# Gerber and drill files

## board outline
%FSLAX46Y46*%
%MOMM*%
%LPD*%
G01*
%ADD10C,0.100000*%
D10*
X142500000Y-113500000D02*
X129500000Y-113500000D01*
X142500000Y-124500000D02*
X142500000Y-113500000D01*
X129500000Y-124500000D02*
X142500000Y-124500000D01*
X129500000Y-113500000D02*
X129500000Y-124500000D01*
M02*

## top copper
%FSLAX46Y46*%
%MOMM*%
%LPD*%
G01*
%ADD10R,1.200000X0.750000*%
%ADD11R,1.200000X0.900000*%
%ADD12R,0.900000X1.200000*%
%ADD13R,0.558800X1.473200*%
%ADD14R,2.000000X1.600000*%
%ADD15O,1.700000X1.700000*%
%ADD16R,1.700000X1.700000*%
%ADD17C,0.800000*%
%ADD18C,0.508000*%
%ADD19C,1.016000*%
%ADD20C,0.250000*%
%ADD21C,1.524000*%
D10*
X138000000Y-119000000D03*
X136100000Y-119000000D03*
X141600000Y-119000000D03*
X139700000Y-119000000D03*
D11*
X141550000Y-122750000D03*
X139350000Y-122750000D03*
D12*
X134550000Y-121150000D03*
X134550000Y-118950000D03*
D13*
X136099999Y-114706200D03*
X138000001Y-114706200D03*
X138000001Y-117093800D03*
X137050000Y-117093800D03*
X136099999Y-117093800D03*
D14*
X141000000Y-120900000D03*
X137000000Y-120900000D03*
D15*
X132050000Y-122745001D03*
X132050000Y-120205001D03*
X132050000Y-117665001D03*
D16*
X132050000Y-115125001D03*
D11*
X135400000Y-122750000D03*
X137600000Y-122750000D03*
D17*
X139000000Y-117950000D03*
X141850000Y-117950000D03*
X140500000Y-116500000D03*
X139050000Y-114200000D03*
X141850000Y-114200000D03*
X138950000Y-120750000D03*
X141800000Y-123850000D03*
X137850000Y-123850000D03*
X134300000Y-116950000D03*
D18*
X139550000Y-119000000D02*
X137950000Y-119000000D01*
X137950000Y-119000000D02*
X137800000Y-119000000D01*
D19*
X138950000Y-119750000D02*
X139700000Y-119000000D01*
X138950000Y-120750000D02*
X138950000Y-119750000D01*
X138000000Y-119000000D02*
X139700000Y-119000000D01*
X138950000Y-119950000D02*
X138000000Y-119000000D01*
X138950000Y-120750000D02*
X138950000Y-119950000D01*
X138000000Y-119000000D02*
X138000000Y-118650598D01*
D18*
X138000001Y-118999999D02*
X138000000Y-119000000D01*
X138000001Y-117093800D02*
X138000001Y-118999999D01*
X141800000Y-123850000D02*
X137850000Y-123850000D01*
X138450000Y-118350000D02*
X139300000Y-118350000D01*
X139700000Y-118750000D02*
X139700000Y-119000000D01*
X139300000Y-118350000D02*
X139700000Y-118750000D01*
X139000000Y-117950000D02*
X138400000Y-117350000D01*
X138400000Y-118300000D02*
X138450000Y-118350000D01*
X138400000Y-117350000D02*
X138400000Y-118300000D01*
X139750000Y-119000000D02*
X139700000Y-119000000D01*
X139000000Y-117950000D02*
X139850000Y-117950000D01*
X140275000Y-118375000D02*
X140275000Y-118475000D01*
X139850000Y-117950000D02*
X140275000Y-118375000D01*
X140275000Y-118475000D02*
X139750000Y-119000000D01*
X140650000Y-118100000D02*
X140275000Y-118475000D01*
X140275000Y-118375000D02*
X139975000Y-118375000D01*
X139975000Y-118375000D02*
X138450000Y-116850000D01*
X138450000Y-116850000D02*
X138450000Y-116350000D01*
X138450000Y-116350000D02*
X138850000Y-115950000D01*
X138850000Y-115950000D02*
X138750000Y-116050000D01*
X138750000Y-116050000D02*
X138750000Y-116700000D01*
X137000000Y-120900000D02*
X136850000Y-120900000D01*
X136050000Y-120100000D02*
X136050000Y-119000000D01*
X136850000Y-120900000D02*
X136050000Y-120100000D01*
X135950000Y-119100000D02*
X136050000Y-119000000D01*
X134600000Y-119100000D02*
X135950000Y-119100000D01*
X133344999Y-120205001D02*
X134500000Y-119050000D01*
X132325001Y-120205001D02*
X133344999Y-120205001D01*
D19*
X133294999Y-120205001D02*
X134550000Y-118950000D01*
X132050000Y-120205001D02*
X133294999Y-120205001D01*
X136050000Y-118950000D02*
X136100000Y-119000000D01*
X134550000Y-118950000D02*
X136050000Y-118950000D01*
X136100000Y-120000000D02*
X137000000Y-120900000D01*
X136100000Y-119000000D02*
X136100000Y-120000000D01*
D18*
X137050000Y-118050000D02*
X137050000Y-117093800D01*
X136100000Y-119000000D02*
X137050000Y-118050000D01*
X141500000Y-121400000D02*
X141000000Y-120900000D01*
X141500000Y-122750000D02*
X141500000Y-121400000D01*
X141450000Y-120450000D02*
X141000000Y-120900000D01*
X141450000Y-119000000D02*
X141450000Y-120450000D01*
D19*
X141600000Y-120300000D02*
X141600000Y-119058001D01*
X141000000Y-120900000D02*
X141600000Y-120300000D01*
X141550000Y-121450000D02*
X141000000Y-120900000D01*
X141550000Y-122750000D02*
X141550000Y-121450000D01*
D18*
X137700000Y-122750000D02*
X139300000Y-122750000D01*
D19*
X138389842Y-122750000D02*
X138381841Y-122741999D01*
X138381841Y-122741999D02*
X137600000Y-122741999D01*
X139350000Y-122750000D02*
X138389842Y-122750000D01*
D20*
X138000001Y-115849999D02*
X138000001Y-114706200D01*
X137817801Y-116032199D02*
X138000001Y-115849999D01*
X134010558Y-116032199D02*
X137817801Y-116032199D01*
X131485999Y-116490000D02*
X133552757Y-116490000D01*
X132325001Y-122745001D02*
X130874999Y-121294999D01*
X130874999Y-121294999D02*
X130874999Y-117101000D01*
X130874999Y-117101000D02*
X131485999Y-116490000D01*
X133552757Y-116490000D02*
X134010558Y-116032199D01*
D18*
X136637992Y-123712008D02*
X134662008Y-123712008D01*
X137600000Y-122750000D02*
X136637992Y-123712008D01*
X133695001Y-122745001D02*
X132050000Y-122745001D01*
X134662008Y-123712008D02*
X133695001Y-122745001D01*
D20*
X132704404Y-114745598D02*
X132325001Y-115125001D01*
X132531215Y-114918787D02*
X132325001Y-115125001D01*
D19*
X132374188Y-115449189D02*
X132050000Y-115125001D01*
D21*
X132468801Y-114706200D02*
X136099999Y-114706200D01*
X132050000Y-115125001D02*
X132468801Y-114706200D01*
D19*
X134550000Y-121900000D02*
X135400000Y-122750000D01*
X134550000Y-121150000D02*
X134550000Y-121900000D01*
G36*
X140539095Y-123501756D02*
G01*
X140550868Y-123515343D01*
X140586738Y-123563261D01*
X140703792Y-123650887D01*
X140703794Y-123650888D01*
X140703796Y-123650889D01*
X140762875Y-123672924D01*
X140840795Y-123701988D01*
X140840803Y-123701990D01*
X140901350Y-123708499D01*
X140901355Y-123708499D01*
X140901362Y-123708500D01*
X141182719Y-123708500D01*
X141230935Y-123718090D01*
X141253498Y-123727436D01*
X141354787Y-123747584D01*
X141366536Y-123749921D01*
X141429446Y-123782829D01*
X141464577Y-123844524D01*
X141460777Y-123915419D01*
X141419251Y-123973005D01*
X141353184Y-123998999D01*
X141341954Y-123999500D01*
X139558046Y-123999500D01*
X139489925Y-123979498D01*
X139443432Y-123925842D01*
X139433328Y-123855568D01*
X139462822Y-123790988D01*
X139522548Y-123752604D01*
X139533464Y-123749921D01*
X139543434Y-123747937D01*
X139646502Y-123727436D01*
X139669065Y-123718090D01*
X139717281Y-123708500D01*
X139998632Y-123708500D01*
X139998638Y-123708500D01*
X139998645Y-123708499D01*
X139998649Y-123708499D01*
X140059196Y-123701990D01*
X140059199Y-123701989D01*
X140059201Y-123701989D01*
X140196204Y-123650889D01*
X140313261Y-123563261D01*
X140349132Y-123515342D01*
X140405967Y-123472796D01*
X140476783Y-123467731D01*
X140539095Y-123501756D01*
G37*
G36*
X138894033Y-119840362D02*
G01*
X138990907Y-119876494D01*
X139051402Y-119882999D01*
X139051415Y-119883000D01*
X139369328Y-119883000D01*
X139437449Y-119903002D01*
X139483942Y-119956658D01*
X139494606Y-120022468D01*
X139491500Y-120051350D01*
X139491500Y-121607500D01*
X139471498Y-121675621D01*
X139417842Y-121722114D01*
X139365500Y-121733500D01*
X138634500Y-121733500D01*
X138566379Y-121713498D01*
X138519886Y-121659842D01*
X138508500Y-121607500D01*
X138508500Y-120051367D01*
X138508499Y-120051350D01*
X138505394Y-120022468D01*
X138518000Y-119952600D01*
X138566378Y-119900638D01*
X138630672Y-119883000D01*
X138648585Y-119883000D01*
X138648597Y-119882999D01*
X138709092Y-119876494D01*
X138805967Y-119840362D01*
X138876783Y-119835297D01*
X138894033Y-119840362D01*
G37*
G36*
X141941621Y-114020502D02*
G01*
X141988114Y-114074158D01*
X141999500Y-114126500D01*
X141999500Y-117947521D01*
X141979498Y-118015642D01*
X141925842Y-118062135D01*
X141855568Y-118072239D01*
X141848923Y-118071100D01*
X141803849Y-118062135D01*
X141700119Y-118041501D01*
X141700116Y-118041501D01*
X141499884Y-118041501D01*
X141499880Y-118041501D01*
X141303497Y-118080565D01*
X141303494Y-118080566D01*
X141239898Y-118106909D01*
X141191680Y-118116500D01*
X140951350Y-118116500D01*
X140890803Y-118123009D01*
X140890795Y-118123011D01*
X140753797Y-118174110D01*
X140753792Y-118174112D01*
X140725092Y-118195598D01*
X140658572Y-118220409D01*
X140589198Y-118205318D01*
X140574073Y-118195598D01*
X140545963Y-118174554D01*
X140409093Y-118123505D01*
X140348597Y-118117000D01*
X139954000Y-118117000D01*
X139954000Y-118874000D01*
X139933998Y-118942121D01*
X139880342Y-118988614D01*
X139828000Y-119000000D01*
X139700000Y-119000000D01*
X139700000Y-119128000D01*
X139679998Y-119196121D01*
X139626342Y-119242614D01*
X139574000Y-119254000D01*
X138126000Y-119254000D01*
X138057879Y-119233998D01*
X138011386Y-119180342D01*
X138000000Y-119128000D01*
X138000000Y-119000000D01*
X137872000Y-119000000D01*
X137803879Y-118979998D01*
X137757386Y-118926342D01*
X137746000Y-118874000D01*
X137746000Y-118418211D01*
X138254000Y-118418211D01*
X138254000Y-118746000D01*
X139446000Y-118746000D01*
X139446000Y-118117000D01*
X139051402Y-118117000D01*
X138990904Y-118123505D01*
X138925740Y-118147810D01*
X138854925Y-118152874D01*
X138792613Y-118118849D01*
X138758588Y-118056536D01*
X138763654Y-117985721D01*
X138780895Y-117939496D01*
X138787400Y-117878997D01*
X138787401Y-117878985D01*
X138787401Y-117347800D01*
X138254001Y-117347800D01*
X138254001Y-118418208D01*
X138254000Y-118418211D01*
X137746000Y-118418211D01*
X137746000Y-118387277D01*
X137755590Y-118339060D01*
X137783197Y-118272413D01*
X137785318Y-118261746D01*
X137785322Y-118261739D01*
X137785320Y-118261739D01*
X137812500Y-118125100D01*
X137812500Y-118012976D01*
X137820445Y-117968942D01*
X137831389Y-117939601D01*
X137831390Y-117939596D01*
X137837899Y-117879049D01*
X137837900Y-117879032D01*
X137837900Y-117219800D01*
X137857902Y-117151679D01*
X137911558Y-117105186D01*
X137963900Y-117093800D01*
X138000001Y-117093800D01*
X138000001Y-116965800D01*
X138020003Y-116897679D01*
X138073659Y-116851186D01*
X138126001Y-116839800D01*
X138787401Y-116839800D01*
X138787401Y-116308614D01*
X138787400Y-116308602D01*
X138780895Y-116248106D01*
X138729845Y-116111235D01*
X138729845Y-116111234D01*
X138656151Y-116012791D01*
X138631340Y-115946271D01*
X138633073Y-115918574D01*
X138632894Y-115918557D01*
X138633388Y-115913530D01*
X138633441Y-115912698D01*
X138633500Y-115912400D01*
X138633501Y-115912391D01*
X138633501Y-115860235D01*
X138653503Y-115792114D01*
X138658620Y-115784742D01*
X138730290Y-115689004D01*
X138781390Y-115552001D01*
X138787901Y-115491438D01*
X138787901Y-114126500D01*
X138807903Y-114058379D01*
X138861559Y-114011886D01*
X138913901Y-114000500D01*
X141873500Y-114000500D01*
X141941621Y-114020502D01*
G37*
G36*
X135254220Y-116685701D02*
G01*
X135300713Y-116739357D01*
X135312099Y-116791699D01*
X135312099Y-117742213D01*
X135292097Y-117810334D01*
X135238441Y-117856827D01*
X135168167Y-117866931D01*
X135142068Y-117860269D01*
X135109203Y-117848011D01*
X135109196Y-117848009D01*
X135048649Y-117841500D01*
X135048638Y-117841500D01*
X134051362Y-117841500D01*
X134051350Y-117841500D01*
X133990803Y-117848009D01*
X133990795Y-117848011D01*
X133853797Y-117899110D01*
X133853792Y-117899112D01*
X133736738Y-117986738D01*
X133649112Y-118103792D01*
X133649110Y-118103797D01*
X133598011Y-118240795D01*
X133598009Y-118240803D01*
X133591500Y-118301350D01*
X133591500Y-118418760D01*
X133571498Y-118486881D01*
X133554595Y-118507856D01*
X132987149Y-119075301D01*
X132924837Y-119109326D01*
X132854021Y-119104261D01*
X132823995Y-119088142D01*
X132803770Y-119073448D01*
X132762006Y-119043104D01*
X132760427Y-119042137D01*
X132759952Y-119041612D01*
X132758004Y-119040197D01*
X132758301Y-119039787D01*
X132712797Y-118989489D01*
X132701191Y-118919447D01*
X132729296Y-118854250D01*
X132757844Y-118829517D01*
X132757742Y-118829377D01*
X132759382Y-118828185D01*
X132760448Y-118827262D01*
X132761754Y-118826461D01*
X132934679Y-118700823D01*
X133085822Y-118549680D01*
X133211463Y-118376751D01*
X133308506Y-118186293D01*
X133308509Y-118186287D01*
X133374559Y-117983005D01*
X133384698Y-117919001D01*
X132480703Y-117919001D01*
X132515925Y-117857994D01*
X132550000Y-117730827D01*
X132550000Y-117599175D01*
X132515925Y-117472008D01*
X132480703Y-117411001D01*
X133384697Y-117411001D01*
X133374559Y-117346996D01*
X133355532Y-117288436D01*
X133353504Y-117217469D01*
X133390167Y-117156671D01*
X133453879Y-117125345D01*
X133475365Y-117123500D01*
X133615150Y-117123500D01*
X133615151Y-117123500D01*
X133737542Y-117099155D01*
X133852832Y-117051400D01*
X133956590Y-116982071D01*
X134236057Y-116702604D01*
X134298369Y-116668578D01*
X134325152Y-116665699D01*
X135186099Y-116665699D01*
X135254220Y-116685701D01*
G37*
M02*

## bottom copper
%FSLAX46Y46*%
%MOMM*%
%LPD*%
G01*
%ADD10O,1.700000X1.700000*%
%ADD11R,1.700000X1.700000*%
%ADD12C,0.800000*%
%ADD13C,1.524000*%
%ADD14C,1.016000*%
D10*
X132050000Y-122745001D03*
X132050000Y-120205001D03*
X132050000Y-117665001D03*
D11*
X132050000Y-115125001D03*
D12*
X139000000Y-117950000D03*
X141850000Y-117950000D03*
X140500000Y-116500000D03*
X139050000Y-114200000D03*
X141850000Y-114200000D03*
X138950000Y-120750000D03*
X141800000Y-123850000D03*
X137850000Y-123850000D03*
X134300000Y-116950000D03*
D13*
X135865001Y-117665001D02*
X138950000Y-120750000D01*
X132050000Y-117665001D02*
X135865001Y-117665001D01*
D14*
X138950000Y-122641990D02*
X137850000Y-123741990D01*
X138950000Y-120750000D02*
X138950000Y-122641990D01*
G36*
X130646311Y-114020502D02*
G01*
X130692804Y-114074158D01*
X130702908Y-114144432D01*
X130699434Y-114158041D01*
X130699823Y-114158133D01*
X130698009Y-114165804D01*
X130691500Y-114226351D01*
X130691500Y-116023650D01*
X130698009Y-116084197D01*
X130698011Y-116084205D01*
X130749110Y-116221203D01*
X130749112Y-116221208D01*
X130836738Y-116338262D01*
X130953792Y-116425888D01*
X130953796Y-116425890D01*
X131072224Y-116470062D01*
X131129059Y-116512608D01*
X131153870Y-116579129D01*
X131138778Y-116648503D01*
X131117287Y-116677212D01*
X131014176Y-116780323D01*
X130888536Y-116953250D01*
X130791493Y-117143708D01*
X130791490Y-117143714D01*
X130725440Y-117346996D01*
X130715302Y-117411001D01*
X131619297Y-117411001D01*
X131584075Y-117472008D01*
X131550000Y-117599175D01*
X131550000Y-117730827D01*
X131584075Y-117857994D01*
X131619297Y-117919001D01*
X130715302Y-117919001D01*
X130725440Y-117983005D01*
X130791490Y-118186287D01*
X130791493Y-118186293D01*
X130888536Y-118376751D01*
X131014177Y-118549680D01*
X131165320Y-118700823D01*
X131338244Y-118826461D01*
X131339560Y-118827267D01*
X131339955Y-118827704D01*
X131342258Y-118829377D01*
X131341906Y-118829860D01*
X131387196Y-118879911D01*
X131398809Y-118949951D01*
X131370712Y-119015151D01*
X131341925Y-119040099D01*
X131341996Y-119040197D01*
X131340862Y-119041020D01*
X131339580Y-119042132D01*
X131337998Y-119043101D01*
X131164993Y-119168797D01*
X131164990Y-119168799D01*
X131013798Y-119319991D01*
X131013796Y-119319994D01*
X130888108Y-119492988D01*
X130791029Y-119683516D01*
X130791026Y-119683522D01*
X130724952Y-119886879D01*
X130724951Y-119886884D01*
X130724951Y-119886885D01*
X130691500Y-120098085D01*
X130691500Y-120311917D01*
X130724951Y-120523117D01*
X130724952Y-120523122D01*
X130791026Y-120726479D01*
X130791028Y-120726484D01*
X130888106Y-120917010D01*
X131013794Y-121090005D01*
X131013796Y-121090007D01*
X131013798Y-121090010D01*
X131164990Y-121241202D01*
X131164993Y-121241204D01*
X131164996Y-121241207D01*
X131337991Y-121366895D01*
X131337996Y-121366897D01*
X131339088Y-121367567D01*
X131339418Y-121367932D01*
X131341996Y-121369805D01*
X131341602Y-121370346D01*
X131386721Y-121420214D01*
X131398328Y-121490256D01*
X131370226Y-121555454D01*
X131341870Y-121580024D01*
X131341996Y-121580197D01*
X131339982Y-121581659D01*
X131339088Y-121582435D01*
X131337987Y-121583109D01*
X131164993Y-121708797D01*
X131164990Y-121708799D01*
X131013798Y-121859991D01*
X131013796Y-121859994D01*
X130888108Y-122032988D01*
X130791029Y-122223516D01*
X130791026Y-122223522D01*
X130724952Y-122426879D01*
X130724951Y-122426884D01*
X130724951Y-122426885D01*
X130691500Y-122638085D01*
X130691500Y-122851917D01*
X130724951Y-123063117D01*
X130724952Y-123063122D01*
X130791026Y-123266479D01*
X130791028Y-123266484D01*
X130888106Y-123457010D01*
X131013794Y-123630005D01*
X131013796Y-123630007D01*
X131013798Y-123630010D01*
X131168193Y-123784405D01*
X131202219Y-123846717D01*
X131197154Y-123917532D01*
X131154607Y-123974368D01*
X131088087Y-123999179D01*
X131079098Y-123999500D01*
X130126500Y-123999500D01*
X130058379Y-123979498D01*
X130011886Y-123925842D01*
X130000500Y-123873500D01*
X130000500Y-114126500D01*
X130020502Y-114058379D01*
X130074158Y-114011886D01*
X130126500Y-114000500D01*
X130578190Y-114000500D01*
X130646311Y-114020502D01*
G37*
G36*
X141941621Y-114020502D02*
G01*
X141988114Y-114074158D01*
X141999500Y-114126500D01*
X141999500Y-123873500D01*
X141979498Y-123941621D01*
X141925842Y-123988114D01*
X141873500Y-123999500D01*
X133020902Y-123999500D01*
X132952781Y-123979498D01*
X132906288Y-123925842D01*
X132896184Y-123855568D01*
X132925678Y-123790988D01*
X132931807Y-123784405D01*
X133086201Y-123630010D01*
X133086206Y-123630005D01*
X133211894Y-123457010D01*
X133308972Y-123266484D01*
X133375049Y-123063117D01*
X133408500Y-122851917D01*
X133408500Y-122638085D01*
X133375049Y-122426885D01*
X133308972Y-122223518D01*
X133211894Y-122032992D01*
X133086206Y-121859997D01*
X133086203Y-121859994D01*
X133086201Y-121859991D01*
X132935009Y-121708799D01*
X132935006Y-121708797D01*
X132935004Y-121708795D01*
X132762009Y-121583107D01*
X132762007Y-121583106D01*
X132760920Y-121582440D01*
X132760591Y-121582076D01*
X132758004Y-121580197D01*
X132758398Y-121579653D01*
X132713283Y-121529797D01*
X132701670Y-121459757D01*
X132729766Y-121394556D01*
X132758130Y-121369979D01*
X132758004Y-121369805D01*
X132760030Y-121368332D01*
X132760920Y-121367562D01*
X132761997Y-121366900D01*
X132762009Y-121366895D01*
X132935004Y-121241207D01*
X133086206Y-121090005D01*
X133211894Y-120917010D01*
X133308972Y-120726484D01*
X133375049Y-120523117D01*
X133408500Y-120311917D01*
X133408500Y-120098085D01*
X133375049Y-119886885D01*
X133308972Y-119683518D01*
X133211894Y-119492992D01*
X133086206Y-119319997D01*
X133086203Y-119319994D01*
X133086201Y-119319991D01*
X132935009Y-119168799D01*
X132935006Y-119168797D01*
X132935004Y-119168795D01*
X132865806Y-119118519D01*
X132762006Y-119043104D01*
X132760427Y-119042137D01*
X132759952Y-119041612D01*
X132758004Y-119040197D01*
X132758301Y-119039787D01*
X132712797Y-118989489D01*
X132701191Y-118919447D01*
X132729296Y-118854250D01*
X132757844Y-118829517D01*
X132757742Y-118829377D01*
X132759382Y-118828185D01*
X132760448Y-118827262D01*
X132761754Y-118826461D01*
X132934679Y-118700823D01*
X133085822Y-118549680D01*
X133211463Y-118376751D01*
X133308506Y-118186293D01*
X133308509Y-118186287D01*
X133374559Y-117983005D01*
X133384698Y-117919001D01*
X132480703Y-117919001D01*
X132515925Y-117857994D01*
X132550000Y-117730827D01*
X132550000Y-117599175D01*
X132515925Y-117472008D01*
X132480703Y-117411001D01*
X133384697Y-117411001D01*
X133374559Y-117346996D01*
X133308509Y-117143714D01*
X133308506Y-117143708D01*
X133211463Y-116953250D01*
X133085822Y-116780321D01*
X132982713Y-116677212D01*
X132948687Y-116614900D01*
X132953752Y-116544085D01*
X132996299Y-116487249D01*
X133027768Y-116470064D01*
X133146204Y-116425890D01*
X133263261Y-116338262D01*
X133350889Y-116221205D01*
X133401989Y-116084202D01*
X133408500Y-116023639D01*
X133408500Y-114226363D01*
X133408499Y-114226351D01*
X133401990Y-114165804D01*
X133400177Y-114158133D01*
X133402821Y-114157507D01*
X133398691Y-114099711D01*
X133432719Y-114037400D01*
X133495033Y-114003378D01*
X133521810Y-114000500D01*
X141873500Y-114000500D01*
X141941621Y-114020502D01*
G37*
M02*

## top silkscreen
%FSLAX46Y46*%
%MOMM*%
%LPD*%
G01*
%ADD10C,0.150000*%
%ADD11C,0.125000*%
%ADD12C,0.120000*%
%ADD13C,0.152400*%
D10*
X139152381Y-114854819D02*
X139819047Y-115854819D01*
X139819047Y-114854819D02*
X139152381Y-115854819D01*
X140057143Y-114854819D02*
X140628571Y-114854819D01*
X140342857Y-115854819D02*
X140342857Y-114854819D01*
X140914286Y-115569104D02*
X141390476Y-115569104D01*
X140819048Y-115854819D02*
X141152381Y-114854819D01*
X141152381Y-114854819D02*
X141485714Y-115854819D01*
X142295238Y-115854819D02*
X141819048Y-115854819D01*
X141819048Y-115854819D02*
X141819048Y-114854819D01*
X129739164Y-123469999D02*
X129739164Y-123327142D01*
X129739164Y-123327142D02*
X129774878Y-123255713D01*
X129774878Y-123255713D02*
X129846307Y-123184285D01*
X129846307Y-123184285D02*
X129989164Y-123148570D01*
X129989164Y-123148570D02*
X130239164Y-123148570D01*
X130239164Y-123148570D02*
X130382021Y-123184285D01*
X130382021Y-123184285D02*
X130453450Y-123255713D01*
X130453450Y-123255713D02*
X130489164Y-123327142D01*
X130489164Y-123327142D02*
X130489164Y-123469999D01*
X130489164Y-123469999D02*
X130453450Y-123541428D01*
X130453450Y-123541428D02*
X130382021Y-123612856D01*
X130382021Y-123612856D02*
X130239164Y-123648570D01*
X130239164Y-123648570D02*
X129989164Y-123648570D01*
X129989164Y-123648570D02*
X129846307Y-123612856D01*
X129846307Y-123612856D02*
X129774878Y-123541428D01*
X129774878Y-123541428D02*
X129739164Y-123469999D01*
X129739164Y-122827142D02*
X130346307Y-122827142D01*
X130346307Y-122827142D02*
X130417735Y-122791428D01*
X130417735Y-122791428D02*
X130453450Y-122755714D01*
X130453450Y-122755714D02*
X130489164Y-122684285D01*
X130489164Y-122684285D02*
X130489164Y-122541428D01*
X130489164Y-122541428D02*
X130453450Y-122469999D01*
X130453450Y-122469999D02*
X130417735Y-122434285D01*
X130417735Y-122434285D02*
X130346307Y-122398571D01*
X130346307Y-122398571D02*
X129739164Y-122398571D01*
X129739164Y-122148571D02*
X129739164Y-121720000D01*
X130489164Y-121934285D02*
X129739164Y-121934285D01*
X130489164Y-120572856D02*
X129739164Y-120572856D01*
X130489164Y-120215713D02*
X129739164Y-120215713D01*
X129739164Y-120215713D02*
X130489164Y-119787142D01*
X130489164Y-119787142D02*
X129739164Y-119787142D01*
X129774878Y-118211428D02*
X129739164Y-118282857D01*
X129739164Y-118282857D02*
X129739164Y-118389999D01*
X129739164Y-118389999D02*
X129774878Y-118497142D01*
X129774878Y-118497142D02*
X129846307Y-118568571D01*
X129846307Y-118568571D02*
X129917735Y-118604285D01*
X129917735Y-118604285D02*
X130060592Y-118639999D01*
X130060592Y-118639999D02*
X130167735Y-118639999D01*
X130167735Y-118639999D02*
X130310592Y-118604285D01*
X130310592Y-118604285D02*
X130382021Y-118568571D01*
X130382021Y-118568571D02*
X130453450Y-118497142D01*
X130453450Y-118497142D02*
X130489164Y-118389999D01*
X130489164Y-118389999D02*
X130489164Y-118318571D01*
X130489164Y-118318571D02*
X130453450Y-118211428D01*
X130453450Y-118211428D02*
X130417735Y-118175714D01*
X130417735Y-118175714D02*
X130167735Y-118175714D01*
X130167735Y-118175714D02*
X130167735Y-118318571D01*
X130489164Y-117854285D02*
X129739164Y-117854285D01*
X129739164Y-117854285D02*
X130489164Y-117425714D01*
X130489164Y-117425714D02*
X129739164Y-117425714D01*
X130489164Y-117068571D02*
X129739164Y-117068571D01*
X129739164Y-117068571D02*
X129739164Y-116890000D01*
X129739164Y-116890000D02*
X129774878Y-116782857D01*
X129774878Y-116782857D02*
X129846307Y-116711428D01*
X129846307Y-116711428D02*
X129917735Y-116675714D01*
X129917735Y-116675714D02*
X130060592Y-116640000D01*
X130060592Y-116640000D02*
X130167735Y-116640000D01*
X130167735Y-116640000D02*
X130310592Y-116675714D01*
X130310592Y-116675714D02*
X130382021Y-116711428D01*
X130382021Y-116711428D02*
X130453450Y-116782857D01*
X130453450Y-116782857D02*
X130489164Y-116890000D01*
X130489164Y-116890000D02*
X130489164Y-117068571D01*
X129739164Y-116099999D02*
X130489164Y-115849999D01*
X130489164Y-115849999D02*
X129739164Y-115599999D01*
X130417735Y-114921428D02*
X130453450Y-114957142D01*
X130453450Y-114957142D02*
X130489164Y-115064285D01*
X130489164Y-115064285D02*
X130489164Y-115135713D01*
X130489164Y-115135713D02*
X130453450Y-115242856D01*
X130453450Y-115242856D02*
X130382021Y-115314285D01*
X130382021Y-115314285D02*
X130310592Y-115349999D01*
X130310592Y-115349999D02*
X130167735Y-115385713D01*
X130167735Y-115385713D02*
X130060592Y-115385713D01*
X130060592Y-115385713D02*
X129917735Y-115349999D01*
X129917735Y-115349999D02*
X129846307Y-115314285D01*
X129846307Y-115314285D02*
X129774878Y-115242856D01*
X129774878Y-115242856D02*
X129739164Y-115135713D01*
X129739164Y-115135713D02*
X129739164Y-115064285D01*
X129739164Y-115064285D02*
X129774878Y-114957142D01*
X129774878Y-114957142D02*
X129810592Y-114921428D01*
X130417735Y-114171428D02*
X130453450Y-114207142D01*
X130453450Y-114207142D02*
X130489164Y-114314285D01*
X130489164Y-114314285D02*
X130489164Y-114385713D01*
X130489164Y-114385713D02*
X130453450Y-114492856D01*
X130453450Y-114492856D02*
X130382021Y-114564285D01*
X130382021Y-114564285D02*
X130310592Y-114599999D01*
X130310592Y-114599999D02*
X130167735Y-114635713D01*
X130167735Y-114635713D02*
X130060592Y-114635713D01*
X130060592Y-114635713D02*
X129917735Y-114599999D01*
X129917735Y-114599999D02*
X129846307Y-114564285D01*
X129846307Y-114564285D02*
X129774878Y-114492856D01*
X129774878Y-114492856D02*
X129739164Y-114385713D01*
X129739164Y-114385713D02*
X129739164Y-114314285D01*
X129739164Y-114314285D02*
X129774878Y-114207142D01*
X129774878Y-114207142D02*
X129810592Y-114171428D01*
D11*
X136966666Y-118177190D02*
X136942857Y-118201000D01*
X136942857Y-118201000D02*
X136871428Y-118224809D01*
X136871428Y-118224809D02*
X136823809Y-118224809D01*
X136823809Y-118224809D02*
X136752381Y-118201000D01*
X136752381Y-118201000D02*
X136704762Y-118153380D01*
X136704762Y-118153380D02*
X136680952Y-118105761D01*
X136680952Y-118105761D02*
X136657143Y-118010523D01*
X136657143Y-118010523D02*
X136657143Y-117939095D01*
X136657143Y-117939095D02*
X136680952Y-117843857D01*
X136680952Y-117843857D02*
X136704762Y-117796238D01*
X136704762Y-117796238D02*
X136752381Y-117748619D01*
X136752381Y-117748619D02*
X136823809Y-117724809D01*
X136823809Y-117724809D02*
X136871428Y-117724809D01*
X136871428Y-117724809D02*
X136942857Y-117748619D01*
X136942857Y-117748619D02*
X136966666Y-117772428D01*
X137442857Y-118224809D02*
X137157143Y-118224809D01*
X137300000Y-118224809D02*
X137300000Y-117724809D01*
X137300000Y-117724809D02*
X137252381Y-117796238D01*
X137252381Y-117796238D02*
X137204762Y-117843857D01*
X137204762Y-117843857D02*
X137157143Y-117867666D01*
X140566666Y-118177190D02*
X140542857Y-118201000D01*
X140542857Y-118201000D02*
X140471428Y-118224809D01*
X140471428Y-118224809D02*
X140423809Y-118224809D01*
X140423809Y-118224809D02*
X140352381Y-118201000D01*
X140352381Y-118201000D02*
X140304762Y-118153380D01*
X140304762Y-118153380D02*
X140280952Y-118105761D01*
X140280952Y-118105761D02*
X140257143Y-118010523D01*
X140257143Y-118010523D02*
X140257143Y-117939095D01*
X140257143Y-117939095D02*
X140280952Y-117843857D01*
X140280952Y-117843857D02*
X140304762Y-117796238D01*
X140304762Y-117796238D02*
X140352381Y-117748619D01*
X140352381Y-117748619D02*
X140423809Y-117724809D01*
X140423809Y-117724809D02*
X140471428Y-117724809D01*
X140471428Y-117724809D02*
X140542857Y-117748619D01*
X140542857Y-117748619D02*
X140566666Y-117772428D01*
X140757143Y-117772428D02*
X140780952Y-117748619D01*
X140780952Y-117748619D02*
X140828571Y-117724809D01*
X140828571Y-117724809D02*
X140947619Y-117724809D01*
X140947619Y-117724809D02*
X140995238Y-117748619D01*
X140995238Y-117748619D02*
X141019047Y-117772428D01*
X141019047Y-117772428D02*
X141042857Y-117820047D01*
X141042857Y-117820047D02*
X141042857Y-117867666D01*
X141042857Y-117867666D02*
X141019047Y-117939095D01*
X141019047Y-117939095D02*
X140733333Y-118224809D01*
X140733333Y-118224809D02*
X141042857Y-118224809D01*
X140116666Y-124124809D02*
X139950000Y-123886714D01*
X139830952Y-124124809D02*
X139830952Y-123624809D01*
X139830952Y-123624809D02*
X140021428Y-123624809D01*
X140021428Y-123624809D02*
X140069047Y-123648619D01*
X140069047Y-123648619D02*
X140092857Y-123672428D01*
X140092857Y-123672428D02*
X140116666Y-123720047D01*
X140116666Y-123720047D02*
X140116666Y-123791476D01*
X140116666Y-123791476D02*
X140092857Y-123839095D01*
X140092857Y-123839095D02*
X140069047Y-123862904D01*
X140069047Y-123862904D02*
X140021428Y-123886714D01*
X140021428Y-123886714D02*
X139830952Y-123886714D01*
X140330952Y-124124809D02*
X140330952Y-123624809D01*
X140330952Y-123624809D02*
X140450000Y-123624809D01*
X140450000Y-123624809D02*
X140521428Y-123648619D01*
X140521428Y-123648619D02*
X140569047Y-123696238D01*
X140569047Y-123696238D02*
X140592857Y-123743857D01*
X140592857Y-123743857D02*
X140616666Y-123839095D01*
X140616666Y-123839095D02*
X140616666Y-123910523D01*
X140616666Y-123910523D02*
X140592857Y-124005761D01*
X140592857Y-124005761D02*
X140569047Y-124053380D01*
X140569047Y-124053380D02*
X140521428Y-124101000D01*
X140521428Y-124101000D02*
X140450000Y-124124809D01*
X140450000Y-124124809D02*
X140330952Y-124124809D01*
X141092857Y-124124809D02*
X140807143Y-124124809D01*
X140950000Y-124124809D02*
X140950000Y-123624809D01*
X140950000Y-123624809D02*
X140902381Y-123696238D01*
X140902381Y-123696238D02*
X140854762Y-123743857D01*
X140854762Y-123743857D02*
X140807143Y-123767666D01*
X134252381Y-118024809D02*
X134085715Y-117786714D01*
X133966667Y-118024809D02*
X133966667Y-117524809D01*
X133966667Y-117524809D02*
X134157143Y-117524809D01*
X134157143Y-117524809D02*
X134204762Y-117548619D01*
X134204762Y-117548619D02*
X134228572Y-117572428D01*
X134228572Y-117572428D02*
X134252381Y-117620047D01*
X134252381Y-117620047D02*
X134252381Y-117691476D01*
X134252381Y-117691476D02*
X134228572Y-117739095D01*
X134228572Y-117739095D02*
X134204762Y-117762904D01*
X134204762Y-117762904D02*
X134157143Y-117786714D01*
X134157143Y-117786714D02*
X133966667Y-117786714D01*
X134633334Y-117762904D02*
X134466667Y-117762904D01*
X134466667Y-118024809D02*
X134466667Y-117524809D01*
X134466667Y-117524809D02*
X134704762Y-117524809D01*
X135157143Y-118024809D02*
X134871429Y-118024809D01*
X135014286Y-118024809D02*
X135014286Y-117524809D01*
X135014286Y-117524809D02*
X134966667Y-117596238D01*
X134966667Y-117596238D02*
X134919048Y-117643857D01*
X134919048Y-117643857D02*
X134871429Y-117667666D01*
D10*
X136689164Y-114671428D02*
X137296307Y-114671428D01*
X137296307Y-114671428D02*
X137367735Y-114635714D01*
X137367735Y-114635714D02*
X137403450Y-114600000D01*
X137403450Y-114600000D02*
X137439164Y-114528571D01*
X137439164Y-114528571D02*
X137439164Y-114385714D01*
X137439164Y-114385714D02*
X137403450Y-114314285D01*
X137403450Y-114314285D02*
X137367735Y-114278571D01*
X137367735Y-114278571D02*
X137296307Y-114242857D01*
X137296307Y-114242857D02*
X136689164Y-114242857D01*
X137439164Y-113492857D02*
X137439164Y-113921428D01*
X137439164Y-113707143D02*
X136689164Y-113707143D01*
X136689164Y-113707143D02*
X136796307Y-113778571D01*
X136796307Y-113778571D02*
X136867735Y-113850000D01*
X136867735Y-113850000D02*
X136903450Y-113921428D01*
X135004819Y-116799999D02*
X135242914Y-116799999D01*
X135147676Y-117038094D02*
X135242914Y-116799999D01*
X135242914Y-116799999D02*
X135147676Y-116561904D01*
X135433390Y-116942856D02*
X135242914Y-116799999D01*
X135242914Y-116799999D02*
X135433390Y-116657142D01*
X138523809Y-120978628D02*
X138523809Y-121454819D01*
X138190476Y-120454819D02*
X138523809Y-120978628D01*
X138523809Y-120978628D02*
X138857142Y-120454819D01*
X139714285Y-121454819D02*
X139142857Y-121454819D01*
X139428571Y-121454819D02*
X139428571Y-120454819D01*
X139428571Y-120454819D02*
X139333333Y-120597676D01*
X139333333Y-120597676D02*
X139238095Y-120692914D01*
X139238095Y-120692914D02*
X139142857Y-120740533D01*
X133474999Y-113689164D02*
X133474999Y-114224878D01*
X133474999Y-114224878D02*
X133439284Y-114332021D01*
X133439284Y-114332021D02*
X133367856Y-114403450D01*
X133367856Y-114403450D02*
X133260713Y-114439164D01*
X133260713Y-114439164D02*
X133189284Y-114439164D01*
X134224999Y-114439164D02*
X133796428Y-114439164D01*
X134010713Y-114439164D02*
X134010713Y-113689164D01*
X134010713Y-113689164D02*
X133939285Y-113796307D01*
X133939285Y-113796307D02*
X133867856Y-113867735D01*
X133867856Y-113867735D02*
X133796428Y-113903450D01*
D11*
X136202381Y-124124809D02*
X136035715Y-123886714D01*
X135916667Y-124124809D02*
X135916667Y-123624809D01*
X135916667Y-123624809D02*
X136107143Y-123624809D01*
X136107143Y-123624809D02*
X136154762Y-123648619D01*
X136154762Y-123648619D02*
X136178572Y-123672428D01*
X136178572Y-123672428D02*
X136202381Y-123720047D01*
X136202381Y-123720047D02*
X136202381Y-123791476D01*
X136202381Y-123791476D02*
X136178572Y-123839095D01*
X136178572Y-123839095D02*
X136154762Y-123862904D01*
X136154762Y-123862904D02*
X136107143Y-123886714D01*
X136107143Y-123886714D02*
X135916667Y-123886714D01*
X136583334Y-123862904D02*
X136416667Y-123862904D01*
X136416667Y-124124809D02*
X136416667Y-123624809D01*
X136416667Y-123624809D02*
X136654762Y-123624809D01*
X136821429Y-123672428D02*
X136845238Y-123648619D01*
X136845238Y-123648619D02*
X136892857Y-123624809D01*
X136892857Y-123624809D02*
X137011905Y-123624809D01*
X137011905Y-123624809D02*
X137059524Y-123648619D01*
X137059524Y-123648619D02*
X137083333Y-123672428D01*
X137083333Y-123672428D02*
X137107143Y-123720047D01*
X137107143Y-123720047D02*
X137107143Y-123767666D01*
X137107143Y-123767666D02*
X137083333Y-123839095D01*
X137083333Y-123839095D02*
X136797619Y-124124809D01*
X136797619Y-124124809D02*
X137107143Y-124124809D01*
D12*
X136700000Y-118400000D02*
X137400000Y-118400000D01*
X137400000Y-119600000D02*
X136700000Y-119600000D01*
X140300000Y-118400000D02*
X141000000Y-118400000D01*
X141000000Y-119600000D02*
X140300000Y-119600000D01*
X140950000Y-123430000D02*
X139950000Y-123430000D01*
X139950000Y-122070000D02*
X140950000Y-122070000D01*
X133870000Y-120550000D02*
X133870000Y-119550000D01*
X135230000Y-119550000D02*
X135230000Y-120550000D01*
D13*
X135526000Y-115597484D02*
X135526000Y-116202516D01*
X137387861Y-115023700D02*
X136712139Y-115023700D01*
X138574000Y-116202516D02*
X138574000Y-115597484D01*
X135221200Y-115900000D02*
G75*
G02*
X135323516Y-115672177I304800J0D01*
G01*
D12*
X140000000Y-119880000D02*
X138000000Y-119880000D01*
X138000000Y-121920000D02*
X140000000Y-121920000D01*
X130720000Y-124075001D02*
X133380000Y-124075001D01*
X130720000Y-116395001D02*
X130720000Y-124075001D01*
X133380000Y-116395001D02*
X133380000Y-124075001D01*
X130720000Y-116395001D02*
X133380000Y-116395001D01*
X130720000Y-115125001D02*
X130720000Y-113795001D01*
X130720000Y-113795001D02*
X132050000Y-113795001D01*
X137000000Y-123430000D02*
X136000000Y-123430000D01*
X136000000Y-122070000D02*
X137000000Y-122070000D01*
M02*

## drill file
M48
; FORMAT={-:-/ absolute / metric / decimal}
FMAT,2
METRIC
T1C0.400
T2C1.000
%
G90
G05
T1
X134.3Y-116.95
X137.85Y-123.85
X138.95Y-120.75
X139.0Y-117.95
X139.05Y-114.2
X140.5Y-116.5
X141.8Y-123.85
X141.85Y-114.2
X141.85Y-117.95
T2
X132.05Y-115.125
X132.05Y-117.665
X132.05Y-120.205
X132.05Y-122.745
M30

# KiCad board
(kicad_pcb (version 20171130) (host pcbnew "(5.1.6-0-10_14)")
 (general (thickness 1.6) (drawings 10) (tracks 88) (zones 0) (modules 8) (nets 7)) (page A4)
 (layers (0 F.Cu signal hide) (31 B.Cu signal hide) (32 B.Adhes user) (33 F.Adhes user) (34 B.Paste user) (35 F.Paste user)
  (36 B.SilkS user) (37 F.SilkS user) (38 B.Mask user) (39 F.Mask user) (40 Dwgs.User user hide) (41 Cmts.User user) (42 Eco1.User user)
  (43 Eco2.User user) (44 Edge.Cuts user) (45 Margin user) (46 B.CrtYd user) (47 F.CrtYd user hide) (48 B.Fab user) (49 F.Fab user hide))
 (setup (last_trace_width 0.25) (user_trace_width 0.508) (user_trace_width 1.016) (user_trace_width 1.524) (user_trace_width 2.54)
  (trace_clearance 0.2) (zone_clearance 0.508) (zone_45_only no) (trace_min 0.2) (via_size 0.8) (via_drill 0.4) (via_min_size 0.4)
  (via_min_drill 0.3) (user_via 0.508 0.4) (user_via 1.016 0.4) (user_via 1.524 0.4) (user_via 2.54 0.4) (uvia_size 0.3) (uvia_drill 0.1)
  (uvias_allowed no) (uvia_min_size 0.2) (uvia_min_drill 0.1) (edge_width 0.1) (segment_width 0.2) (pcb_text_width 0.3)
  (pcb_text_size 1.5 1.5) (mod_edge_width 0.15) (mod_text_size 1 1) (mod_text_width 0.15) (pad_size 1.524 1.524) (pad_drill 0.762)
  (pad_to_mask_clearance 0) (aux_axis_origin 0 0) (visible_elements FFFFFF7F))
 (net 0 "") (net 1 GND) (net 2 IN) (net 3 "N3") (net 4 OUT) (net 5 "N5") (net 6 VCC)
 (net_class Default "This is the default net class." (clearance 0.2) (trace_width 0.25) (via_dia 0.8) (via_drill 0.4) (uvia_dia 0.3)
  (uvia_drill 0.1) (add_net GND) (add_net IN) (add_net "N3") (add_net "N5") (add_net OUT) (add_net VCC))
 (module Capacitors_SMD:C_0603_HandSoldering (layer F.Cu) (at 137.05 119)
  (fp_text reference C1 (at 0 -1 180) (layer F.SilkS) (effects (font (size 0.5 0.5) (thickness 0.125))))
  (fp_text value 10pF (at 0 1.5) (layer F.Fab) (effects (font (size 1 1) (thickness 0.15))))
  (fp_line (start -0.35 -0.6) (end 0.35 -0.6) (layer F.SilkS) (width 0.12))
  (fp_line (start 0.35 0.6) (end -0.35 0.6) (layer F.SilkS) (width 0.12))
  (pad 2 smd rect (at 0.95 0) (size 1.2 0.75) (layers F.Cu F.Paste F.Mask) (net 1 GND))
  (pad 1 smd rect (at -0.95 0) (size 1.2 0.75) (layers F.Cu F.Paste F.Mask) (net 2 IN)))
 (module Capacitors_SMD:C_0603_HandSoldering (layer F.Cu) (at 140.65 119 180)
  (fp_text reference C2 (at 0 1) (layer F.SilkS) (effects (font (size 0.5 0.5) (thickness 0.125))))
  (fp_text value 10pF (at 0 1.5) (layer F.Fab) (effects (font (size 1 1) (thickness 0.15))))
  (fp_line (start 0.35 0.6) (end -0.35 0.6) (layer F.SilkS) (width 0.12))
  (fp_line (start -0.35 -0.6) (end 0.35 -0.6) (layer F.SilkS) (width 0.12))
  (pad 1 smd rect (at -0.95 0 180) (size 1.2 0.75) (layers F.Cu F.Paste F.Mask) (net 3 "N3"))
  (pad 2 smd rect (at 0.95 0 180) (size 1.2 0.75) (layers F.Cu F.Paste F.Mask) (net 1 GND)))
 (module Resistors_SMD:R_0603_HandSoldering (layer F.Cu) (at 140.45 122.75)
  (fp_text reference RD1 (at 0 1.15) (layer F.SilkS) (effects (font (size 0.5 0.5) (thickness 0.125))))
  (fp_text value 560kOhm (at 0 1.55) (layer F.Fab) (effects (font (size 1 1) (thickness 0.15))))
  (fp_line (start 0.5 0.68) (end -0.5 0.68) (layer F.SilkS) (width 0.12))
  (fp_line (start -0.5 -0.68) (end 0.5 -0.68) (layer F.SilkS) (width 0.12))
  (pad 2 smd rect (at 1.1 0) (size 1.2 0.9) (layers F.Cu F.Paste F.Mask) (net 3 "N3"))
  (pad 1 smd rect (at -1.1 0) (size 1.2 0.9) (layers F.Cu F.Paste F.Mask) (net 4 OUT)))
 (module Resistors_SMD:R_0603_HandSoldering (layer F.Cu) (at 134.55 120.05 90)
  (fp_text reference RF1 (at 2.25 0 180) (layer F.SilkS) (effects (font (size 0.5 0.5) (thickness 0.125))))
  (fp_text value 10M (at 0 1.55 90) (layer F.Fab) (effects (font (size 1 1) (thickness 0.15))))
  (fp_line (start -0.5 -0.68) (end 0.5 -0.68) (layer F.SilkS) (width 0.12))
  (fp_line (start 0.5 0.68) (end -0.5 0.68) (layer F.SilkS) (width 0.12))
  (pad 1 smd rect (at -1.1 0 90) (size 1.2 0.9) (layers F.Cu F.Paste F.Mask) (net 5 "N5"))
  (pad 2 smd rect (at 1.1 0 90) (size 1.2 0.9) (layers F.Cu F.Paste F.Mask) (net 2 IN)))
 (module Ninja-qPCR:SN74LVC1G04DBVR (layer F.Cu) (at 137.05 115.9 90)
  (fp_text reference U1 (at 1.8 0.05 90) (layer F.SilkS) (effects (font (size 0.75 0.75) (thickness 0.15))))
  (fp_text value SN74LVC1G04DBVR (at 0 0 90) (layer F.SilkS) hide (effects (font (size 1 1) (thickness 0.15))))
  (fp_line (start 0.302516 -1.524) (end -0.302516 -1.524) (layer F.SilkS) (width 0.1524))
  (fp_line (start 0.8763 0.337861) (end 0.8763 -0.337861) (layer F.SilkS) (width 0.1524))
  (fp_line (start -0.302516 1.524) (end 0.302516 1.524) (layer F.SilkS) (width 0.1524))
  (fp_arc (start 0 -1.524) (end 0 -1.8288) (angle 48.370041) (layer F.SilkS) (width 0.1524))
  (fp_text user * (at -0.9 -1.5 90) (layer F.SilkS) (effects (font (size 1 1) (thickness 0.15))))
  (pad 5 smd rect (at 1.1938 -0.950001 90) (size 1.4732 0.5588) (layers F.Cu F.Paste F.Mask) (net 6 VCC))
  (pad 4 smd rect (at 1.1938 0.950001 90) (size 1.4732 0.5588) (layers F.Cu F.Paste F.Mask) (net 4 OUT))
  (pad 3 smd rect (at -1.1938 0.950001 90) (size 1.4732 0.5588) (layers F.Cu F.Paste F.Mask) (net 1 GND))
  (pad 2 smd rect (at -1.1938 0 90) (size 1.4732 0.5588) (layers F.Cu F.Paste F.Mask) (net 2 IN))
  (pad 1 smd rect (at -1.1938 -0.950001 90) (size 1.4732 0.5588) (layers F.Cu F.Paste F.Mask)))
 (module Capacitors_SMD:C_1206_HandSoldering (layer F.Cu) (at 139 120.9)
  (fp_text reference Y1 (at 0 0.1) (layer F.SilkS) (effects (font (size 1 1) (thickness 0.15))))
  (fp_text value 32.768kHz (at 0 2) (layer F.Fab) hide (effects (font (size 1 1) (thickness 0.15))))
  (fp_line (start 1 -1.02) (end -1 -1.02) (layer F.SilkS) (width 0.12))
  (fp_line (start -1 1.02) (end 1 1.02) (layer F.SilkS) (width 0.12))
  (pad 2 smd rect (at 2 0) (size 2 1.6) (layers F.Cu F.Paste F.Mask) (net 3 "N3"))
  (pad 1 smd rect (at -2 0) (size 2 1.6) (layers F.Cu F.Paste F.Mask) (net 2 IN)))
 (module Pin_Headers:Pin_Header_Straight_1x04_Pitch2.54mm (layer F.Cu) (at 132.05 115.125001)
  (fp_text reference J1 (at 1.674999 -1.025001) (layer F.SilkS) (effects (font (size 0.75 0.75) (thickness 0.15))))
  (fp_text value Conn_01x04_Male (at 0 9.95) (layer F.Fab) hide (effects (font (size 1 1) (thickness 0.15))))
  (fp_line (start -1.33 8.95) (end 1.33 8.95) (layer F.SilkS) (width 0.12))
  (fp_line (start -1.33 1.27) (end -1.33 8.95) (layer F.SilkS) (width 0.12))
  (fp_line (start 1.33 1.27) (end 1.33 8.95) (layer F.SilkS) (width 0.12))
  (fp_line (start -1.33 1.27) (end 1.33 1.27) (layer F.SilkS) (width 0.12))
  (fp_line (start -1.33 0) (end -1.33 -1.33) (layer F.SilkS) (width 0.12))
  (fp_line (start -1.33 -1.33) (end 0 -1.33) (layer F.SilkS) (width 0.12))
  (pad 4 thru_hole oval (at 0 7.62) (size 1.7 1.7) (drill 1) (layers *.Cu *.Mask) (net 4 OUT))
  (pad 3 thru_hole oval (at 0 5.08) (size 1.7 1.7) (drill 1) (layers *.Cu *.Mask) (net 2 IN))
  (pad 2 thru_hole oval (at 0 2.54) (size 1.7 1.7) (drill 1) (layers *.Cu *.Mask) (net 1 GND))
  (pad 1 thru_hole rect (at 0 0) (size 1.7 1.7) (drill 1) (layers *.Cu *.Mask) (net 6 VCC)))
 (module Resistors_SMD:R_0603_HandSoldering (layer F.Cu) (at 136.5 122.75 180)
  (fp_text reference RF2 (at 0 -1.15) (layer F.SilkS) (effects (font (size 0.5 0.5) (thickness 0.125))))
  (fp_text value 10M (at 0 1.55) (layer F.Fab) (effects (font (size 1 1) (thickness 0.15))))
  (fp_line (start -0.5 -0.68) (end 0.5 -0.68) (layer F.SilkS) (width 0.12))
  (fp_line (start 0.5 0.68) (end -0.5 0.68) (layer F.SilkS) (width 0.12))
  (pad 2 smd rect (at 1.1 0 180) (size 1.2 0.9) (layers F.Cu F.Paste F.Mask) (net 5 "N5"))
  (pad 1 smd rect (at -1.1 0 180) (size 1.2 0.9) (layers F.Cu F.Paste F.Mask) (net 4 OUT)))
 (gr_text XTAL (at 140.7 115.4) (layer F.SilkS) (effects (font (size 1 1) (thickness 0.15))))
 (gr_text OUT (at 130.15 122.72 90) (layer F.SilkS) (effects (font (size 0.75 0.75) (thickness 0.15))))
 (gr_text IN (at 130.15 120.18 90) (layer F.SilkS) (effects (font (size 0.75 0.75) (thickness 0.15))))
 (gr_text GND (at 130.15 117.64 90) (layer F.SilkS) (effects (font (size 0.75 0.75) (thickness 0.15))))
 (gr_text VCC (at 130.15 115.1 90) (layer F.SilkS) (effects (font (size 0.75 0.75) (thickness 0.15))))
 (gr_line (start 142.5 113.5) (end 129.5 113.5) (layer Edge.Cuts) (width 0.1))
 (gr_line (start 142.5 124.5) (end 142.5 113.5) (layer Edge.Cuts) (width 0.1))
 (gr_line (start 129.5 124.5) (end 142.5 124.5) (layer Edge.Cuts) (width 0.1))
 (gr_line (start 129.5 113.5) (end 129.5 124.5) (layer Edge.Cuts) (width 0.1))
 (via (at 139 117.95) (size 0.8) (drill 0.4) (layers F.Cu B.Cu) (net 1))
 (via (at 141.85 117.95) (size 0.8) (drill 0.4) (layers F.Cu B.Cu) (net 1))
 (via (at 140.5 116.5) (size 0.8) (drill 0.4) (layers F.Cu B.Cu) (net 1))
 (via (at 139.05 114.2) (size 0.8) (drill 0.4) (layers F.Cu B.Cu) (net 1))
 (via (at 141.85 114.2) (size 0.8) (drill 0.4) (layers F.Cu B.Cu) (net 1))
 (via (at 138.95 120.75) (size 0.8) (drill 0.4) (layers F.Cu B.Cu) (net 1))
 (segment (start 139.55 119) (end 137.95 119) (width 0.508) (layer F.Cu) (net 1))
 (segment (start 137.95 119) (end 137.8 119) (width 0.508) (layer F.Cu) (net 1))
 (via (at 141.8 123.85) (size 0.8) (drill 0.4) (layers F.Cu B.Cu) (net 1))
 (via (at 137.85 123.85) (size 0.8) (drill 0.4) (layers F.Cu B.Cu) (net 1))
 (segment (start 135.865001 117.665001) (end 138.95 120.75) (width 1.524) (layer B.Cu) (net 1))
 (segment (start 132.05 117.665001) (end 135.865001 117.665001) (width 1.524) (layer B.Cu) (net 1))
 (segment (start 138.95 119.75) (end 139.7 119) (width 1.016) (layer F.Cu) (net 1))
 (segment (start 138.95 120.75) (end 138.95 119.75) (width 1.016) (layer F.Cu) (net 1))
 (segment (start 138 119) (end 139.7 119) (width 1.016) (layer F.Cu) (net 1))
 (segment (start 138.95 119.95) (end 138 119) (width 1.016) (layer F.Cu) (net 1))
 (segment (start 138.95 120.75) (end 138.95 119.95) (width 1.016) (layer F.Cu) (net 1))
 (segment (start 138 119) (end 138 118.650598) (width 1.016) (layer F.Cu) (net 1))
 (segment (start 138.95 122.64199) (end 137.85 123.74199) (width 1.016) (layer B.Cu) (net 1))
 (segment (start 138.95 120.75) (end 138.95 122.64199) (width 1.016) (layer B.Cu) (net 1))
 (segment (start 138.000001 118.999999) (end 138 119) (width 0.508) (layer F.Cu) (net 1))
 (segment (start 138.000001 117.0938) (end 138.000001 118.999999) (width 0.508) (layer F.Cu) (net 1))
 (segment (start 141.8 123.85) (end 137.85 123.85) (width 0.508) (layer F.Cu) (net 1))
 (segment (start 138.45 118.35) (end 139.3 118.35) (width 0.508) (layer F.Cu) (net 1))
 (segment (start 139.7 118.75) (end 139.7 119) (width 0.508) (layer F.Cu) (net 1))
 (segment (start 139.3 118.35) (end 139.7 118.75) (width 0.508) (layer F.Cu) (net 1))
 (segment (start 139 117.95) (end 138.4 117.35) (width 0.508) (layer F.Cu) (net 1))
 (segment (start 138.4 118.3) (end 138.45 118.35) (width 0.508) (layer F.Cu) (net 1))
 (segment (start 138.4 117.35) (end 138.4 118.3) (width 0.508) (layer F.Cu) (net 1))
 (segment (start 139.75 119) (end 139.7 119) (width 0.508) (layer F.Cu) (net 1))
 (segment (start 139 117.95) (end 139.85 117.95) (width 0.508) (layer F.Cu) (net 1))
 (segment (start 140.275 118.375) (end 140.275 118.475) (width 0.508) (layer F.Cu) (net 1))
 (segment (start 139.85 117.95) (end 140.275 118.375) (width 0.508) (layer F.Cu) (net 1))
 (segment (start 140.275 118.475) (end 139.75 119) (width 0.508) (layer F.Cu) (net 1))
 (segment (start 140.65 118.1) (end 140.275 118.475) (width 0.508) (layer F.Cu) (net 1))
 (segment (start 140.275 118.375) (end 139.975 118.375) (width 0.508) (layer F.Cu) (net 1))
 (segment (start 139.975 118.375) (end 138.45 116.85) (width 0.508) (layer F.Cu) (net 1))
 (segment (start 138.45 116.85) (end 138.45 116.35) (width 0.508) (layer F.Cu) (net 1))
 (segment (start 138.45 116.35) (end 138.85 115.95) (width 0.508) (layer F.Cu) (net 1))
 (segment (start 138.85 115.95) (end 138.75 116.05) (width 0.508) (layer F.Cu) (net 1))
 (segment (start 138.75 116.05) (end 138.75 116.7) (width 0.508) (layer F.Cu) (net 1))
 (via (at 134.3 116.95) (size 0.8) (drill 0.4) (layers F.Cu B.Cu) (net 1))
 (segment (start 137 120.9) (end 136.85 120.9) (width 0.508) (layer F.Cu) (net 2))
 (segment (start 136.05 120.1) (end 136.05 119) (width 0.508) (layer F.Cu) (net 2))
 (segment (start 136.85 120.9) (end 136.05 120.1) (width 0.508) (layer F.Cu) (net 2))
 (segment (start 135.95 119.1) (end 136.05 119) (width 0.508) (layer F.Cu) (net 2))
 (segment (start 134.6 119.1) (end 135.95 119.1) (width 0.508) (layer F.Cu) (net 2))
 (segment (start 133.344999 120.205001) (end 134.5 119.05) (width 0.508) (layer F.Cu) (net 2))
 (segment (start 132.325001 120.205001) (end 133.344999 120.205001) (width 0.508) (layer F.Cu) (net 2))
 (segment (start 133.294999 120.205001) (end 134.55 118.95) (width 1.016) (layer F.Cu) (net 2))
 (segment (start 132.05 120.205001) (end 133.294999 120.205001) (width 1.016) (layer F.Cu) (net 2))
 (segment (start 136.05 118.95) (end 136.1 119) (width 1.016) (layer F.Cu) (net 2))
 (segment (start 134.55 118.95) (end 136.05 118.95) (width 1.016) (layer F.Cu) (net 2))
 (segment (start 136.1 120) (end 137 120.9) (width 1.016) (layer F.Cu) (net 2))
 (segment (start 136.1 119) (end 136.1 120) (width 1.016) (layer F.Cu) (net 2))
 (segment (start 137.05 118.05) (end 137.05 117.0938) (width 0.508) (layer F.Cu) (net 2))
 (segment (start 136.1 119) (end 137.05 118.05) (width 0.508) (layer F.Cu) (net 2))
 (segment (start 141.5 121.4) (end 141 120.9) (width 0.508) (layer F.Cu) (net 3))
 (segment (start 141.5 122.75) (end 141.5 121.4) (width 0.508) (layer F.Cu) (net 3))
 (segment (start 141.45 120.45) (end 141 120.9) (width 0.508) (layer F.Cu) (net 3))
 (segment (start 141.45 119) (end 141.45 120.45) (width 0.508) (layer F.Cu) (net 3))
 (segment (start 141.6 120.3) (end 141.6 119.058001) (width 1.016) (layer F.Cu) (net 3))
 (segment (start 141 120.9) (end 141.6 120.3) (width 1.016) (layer F.Cu) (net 3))
 (segment (start 141.55 121.45) (end 141 120.9) (width 1.016) (layer F.Cu) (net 3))
 (segment (start 141.55 122.75) (end 141.55 121.45) (width 1.016) (layer F.Cu) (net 3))
 (segment (start 137.7 122.75) (end 139.3 122.75) (width 0.508) (layer F.Cu) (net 4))
 (segment (start 138.389842 122.75) (end 138.381841 122.741999) (width 1.016) (layer F.Cu) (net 4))
 (segment (start 138.381841 122.741999) (end 137.6 122.741999) (width 1.016) (layer F.Cu) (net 4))
 (segment (start 139.35 122.75) (end 138.389842 122.75) (width 1.016) (layer F.Cu) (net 4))
 (segment (start 138.000001 115.849999) (end 138.000001 114.7062) (width 0.25) (layer F.Cu) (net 4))
 (segment (start 137.817801 116.032199) (end 138.000001 115.849999) (width 0.25) (layer F.Cu) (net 4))
 (segment (start 134.010558 116.032199) (end 137.817801 116.032199) (width 0.25) (layer F.Cu) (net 4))
 (segment (start 131.485999 116.49) (end 133.552757 116.49) (width 0.25) (layer F.Cu) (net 4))
 (segment (start 132.325001 122.745001) (end 130.874999 121.294999) (width 0.25) (layer F.Cu) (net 4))
 (segment (start 130.874999 121.294999) (end 130.874999 117.101) (width 0.25) (layer F.Cu) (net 4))
 (segment (start 130.874999 117.101) (end 131.485999 116.49) (width 0.25) (layer F.Cu) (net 4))
 (segment (start 133.552757 116.49) (end 134.010558 116.032199) (width 0.25) (layer F.Cu) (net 4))
 (segment (start 136.637992 123.712008) (end 134.662008 123.712008) (width 0.508) (layer F.Cu) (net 4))
 (segment (start 137.6 122.75) (end 136.637992 123.712008) (width 0.508) (layer F.Cu) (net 4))
 (segment (start 133.695001 122.745001) (end 132.05 122.745001) (width 0.508) (layer F.Cu) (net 4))
 (segment (start 134.662008 123.712008) (end 133.695001 122.745001) (width 0.508) (layer F.Cu) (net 4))
 (segment (start 132.704404 114.745598) (end 132.325001 115.125001) (width 0.25) (layer F.Cu) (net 6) (status 30))
 (segment (start 132.531215 114.918787) (end 132.325001 115.125001) (width 0.25) (layer F.Cu) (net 6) (status 30))
 (segment (start 132.374188 115.449189) (end 132.05 115.125001) (width 1.016) (layer F.Cu) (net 6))
 (segment (start 132.468801 114.7062) (end 136.099999 114.7062) (width 1.524) (layer F.Cu) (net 6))
 (segment (start 132.05 115.125001) (end 132.468801 114.7062) (width 1.524) (layer F.Cu) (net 6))
 (segment (start 134.55 121.9) (end 135.4 122.75) (width 1.016) (layer F.Cu) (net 5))
 (segment (start 134.55 121.15) (end 134.55 121.9) (width 1.016) (layer F.Cu) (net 5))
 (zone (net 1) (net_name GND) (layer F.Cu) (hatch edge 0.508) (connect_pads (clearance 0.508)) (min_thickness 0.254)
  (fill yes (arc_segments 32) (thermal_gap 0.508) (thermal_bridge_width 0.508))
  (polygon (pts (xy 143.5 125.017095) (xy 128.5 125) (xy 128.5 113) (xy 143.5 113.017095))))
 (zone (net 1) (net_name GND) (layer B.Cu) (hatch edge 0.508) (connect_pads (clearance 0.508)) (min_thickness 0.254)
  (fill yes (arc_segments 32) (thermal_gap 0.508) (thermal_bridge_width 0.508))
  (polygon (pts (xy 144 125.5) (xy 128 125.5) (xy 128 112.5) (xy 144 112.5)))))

